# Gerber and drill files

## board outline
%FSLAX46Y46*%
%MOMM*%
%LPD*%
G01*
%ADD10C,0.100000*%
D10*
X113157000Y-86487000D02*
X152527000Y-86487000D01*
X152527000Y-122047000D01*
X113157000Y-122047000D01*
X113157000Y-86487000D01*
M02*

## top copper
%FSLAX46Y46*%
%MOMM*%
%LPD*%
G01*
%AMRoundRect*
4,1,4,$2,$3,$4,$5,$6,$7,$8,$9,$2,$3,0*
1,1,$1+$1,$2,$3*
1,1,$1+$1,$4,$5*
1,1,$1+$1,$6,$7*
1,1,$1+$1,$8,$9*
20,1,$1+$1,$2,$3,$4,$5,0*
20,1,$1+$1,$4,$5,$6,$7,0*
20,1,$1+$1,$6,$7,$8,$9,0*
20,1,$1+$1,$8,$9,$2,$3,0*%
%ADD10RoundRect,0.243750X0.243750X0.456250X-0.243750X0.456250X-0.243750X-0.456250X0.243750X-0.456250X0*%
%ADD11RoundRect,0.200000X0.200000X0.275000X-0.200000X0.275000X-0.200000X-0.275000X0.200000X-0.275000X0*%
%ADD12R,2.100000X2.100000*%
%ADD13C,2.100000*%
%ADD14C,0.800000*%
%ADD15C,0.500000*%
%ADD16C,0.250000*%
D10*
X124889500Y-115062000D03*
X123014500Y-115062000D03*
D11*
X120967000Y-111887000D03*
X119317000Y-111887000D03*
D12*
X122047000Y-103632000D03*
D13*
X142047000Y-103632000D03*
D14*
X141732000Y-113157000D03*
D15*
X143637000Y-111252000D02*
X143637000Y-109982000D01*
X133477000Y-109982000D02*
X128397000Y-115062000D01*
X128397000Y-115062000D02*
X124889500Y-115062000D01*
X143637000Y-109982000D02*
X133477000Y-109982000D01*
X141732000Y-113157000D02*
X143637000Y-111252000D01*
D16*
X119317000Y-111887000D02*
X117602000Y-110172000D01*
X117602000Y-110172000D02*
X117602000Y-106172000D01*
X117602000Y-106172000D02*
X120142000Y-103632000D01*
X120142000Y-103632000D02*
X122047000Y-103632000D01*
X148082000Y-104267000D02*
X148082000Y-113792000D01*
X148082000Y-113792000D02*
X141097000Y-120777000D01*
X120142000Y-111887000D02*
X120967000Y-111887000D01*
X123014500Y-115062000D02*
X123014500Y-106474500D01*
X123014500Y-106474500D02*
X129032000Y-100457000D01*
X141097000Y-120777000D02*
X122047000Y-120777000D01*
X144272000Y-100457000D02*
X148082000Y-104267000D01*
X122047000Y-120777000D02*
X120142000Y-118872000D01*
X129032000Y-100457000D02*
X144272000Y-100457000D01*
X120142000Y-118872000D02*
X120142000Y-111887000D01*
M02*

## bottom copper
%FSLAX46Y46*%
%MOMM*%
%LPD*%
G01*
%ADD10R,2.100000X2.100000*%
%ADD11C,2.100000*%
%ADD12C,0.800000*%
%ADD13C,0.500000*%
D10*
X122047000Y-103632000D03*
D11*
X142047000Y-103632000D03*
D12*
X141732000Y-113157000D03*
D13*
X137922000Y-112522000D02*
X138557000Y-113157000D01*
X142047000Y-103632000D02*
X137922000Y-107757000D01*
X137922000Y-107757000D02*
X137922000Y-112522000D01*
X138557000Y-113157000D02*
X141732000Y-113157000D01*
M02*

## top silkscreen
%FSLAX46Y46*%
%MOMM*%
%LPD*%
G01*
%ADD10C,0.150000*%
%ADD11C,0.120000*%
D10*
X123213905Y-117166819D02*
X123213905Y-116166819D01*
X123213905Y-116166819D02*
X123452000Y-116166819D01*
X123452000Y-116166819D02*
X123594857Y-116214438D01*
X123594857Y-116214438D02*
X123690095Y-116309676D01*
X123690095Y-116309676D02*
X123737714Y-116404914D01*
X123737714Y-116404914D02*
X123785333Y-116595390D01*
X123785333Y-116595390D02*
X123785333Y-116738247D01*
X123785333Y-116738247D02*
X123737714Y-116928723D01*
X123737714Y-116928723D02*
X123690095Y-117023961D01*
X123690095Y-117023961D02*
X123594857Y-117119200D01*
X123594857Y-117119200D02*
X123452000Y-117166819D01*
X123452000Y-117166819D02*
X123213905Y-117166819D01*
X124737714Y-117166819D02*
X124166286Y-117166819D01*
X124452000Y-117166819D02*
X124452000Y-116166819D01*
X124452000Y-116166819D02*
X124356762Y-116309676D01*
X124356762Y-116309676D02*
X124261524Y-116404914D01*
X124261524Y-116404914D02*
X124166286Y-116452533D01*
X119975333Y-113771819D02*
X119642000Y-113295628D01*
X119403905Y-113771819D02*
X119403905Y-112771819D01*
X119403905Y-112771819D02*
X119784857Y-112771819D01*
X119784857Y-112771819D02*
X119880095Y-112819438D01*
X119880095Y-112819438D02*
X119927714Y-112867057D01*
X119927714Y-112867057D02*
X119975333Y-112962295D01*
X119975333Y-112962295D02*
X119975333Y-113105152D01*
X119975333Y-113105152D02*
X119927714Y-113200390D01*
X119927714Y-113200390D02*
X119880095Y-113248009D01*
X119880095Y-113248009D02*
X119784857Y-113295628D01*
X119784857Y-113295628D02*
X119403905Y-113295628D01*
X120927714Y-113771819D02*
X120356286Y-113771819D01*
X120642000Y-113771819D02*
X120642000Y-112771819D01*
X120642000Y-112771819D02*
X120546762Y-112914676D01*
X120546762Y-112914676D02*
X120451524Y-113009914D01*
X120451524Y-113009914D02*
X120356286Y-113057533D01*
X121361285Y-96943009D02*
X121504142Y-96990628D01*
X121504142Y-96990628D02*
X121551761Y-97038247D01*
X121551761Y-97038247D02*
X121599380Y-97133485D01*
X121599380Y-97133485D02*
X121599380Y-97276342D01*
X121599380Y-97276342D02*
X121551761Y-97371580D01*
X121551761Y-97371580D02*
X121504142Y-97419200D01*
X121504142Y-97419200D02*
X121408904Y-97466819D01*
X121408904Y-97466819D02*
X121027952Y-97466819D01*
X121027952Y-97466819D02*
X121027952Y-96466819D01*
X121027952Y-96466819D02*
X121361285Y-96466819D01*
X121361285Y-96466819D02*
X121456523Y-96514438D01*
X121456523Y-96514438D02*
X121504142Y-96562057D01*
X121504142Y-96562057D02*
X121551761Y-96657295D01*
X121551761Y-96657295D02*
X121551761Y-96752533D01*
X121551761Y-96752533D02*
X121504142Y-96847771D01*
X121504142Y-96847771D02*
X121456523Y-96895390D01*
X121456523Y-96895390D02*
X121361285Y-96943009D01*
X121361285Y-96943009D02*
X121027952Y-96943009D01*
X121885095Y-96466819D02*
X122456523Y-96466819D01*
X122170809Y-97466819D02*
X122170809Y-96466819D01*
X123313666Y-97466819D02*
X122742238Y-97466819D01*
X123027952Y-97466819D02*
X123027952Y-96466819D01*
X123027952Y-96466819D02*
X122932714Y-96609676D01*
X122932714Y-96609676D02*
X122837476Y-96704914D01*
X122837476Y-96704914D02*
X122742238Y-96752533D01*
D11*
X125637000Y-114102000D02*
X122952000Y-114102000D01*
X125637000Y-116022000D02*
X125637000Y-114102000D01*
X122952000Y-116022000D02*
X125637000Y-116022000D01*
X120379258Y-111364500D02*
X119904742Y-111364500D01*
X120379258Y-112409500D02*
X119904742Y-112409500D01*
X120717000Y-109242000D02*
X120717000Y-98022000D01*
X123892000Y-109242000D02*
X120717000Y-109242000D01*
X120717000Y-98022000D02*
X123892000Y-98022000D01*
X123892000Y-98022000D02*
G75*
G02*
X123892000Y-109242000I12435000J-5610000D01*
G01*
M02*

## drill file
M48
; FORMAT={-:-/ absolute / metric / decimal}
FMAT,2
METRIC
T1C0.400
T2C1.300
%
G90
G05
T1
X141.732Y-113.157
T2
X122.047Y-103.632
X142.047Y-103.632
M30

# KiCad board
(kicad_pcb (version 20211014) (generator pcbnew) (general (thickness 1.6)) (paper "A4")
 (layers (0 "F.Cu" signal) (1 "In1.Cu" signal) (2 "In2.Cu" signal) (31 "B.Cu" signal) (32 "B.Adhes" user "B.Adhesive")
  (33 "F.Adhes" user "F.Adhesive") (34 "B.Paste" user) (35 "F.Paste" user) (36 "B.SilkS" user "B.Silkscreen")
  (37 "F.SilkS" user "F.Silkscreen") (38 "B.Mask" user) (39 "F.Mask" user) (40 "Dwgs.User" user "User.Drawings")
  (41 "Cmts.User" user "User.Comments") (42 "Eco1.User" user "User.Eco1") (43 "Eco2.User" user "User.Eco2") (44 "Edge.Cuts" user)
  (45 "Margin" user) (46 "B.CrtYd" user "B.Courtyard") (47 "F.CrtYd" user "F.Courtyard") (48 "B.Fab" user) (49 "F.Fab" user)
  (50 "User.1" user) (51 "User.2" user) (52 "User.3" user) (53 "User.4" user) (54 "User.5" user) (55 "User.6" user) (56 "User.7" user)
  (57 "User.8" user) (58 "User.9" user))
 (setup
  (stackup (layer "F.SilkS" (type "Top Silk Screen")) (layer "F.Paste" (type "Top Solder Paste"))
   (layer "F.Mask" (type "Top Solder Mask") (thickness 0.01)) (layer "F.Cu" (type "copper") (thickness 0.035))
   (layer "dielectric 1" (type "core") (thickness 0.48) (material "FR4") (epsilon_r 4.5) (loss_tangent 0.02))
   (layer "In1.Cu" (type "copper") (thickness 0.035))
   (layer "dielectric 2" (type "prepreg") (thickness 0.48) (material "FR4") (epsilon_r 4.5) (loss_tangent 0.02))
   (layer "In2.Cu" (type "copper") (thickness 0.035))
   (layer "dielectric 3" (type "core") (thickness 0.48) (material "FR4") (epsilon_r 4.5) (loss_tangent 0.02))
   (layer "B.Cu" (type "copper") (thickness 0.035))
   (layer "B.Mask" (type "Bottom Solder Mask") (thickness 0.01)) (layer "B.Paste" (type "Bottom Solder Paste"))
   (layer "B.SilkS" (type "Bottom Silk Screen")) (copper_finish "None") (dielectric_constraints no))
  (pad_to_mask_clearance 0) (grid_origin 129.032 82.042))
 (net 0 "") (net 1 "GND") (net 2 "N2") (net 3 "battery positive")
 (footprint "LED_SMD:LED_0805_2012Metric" (layer "F.Cu") (at 123.952 115.062 180)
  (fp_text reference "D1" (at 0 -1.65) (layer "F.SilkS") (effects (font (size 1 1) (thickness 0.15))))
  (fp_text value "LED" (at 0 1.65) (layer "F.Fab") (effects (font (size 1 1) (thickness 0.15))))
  (fp_line (start -1.685 0.96) (end 1 0.96) (layer "F.SilkS") (width 0.12))
  (fp_line (start -1.685 -0.96) (end -1.685 0.96) (layer "F.SilkS") (width 0.12))
  (fp_line (start 1 -0.96) (end -1.685 -0.96) (layer "F.SilkS") (width 0.12))
  (pad "1" smd roundrect (at -0.9375 0 180) (size 0.975 1.4) (layers "F.Cu" "F.Paste" "F.Mask") (roundrect_rratio 0.25) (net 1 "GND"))
  (pad "2" smd roundrect (at 0.9375 0 180) (size 0.975 1.4) (layers "F.Cu" "F.Paste" "F.Mask") (roundrect_rratio 0.25) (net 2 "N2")))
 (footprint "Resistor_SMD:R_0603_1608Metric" (layer "F.Cu") (at 120.142 111.887 180)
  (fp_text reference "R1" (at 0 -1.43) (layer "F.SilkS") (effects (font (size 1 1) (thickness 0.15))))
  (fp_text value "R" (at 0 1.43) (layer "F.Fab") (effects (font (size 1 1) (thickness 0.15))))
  (fp_line (start -0.237258 0.5225) (end 0.237258 0.5225) (layer "F.SilkS") (width 0.12))
  (fp_line (start -0.237258 -0.5225) (end 0.237258 -0.5225) (layer "F.SilkS") (width 0.12))
  (pad "1" smd roundrect (at -0.825 0 180) (size 0.8 0.95) (layers "F.Cu" "F.Paste" "F.Mask") (roundrect_rratio 0.25) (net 2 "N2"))
  (pad "2" smd roundrect (at 0.825 0 180) (size 0.8 0.95) (layers "F.Cu" "F.Paste" "F.Mask") (roundrect_rratio 0.25)
   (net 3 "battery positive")))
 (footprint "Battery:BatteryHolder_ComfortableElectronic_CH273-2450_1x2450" (layer "F.Cu") (at 122.047 103.632)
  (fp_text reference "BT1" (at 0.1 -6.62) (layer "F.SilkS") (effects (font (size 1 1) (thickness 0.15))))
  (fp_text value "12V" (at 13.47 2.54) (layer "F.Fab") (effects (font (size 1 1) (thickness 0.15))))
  (fp_line (start -1.33 5.61) (end -1.33 -5.61) (layer "F.SilkS") (width 0.12))
  (fp_line (start 1.845 5.61) (end -1.33 5.61) (layer "F.SilkS") (width 0.12))
  (fp_line (start -1.33 -5.61) (end 1.845 -5.61) (layer "F.SilkS") (width 0.12))
  (fp_arc (start 1.845 -5.61) (mid 27.921896 0) (end 1.845 5.61) (layer "F.SilkS") (width 0.12))
  (pad "1" thru_hole rect (at 0 0 270) (size 2.1 2.1) (drill 1.3) (layers *.Cu *.Mask) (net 3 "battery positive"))
  (pad "2" thru_hole circle (at 20 0 270) (size 2.1 2.1) (drill 1.3) (layers *.Cu *.Mask) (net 1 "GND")))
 (gr_rect (start 152.527 122.047) (end 113.157 86.487) (layer "Edge.Cuts") (width 0.1) (fill none))
 (segment (start 143.637 111.252) (end 143.637 109.982) (width 0.5) (layer "F.Cu") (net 1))
 (segment (start 133.477 109.982) (end 128.397 115.062) (width 0.5) (layer "F.Cu") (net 1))
 (segment (start 128.397 115.062) (end 124.8895 115.062) (width 0.5) (layer "F.Cu") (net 1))
 (segment (start 143.637 109.982) (end 133.477 109.982) (width 0.5) (layer "F.Cu") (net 1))
 (segment (start 141.732 113.157) (end 143.637 111.252) (width 0.5) (layer "F.Cu") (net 1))
 (via (at 141.732 113.157) (size 0.8) (drill 0.4) (layers "F.Cu" "B.Cu") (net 1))
 (segment (start 137.922 112.522) (end 138.557 113.157) (width 0.5) (layer "B.Cu") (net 1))
 (segment (start 142.047 103.632) (end 137.922 107.757) (width 0.5) (layer "B.Cu") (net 1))
 (segment (start 137.922 107.757) (end 137.922 112.522) (width 0.5) (layer "B.Cu") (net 1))
 (segment (start 138.557 113.157) (end 141.732 113.157) (width 0.5) (layer "B.Cu") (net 1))
 (segment (start 119.317 111.887) (end 117.602 110.172) (width 0.25) (layer "F.Cu") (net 3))
 (segment (start 117.602 110.172) (end 117.602 106.172) (width 0.25) (layer "F.Cu") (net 3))
 (segment (start 117.602 106.172) (end 120.142 103.632) (width 0.25) (layer "F.Cu") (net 3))
 (segment (start 120.142 103.632) (end 122.047 103.632) (width 0.25) (layer "F.Cu") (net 3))
 (segment (start 148.082 104.267) (end 148.082 113.792) (width 0.25) (layer "F.Cu") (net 2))
 (segment (start 148.082 113.792) (end 141.097 120.777) (width 0.25) (layer "F.Cu") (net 2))
 (segment (start 120.142 111.887) (end 120.967 111.887) (width 0.25) (layer "F.Cu") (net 2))
 (segment (start 123.0145 115.062) (end 123.0145 106.4745) (width 0.25) (layer "F.Cu") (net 2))
 (segment (start 123.0145 106.4745) (end 129.032 100.457) (width 0.25) (layer "F.Cu") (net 2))
 (segment (start 141.097 120.777) (end 122.047 120.777) (width 0.25) (layer "F.Cu") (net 2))
 (segment (start 144.272 100.457) (end 148.082 104.267) (width 0.25) (layer "F.Cu") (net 2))
 (segment (start 122.047 120.777) (end 120.142 118.872) (width 0.25) (layer "F.Cu") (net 2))
 (segment (start 129.032 100.457) (end 144.272 100.457) (width 0.25) (layer "F.Cu") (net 2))
 (segment (start 120.142 118.872) (end 120.142 111.887) (width 0.25) (layer "F.Cu") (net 2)))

